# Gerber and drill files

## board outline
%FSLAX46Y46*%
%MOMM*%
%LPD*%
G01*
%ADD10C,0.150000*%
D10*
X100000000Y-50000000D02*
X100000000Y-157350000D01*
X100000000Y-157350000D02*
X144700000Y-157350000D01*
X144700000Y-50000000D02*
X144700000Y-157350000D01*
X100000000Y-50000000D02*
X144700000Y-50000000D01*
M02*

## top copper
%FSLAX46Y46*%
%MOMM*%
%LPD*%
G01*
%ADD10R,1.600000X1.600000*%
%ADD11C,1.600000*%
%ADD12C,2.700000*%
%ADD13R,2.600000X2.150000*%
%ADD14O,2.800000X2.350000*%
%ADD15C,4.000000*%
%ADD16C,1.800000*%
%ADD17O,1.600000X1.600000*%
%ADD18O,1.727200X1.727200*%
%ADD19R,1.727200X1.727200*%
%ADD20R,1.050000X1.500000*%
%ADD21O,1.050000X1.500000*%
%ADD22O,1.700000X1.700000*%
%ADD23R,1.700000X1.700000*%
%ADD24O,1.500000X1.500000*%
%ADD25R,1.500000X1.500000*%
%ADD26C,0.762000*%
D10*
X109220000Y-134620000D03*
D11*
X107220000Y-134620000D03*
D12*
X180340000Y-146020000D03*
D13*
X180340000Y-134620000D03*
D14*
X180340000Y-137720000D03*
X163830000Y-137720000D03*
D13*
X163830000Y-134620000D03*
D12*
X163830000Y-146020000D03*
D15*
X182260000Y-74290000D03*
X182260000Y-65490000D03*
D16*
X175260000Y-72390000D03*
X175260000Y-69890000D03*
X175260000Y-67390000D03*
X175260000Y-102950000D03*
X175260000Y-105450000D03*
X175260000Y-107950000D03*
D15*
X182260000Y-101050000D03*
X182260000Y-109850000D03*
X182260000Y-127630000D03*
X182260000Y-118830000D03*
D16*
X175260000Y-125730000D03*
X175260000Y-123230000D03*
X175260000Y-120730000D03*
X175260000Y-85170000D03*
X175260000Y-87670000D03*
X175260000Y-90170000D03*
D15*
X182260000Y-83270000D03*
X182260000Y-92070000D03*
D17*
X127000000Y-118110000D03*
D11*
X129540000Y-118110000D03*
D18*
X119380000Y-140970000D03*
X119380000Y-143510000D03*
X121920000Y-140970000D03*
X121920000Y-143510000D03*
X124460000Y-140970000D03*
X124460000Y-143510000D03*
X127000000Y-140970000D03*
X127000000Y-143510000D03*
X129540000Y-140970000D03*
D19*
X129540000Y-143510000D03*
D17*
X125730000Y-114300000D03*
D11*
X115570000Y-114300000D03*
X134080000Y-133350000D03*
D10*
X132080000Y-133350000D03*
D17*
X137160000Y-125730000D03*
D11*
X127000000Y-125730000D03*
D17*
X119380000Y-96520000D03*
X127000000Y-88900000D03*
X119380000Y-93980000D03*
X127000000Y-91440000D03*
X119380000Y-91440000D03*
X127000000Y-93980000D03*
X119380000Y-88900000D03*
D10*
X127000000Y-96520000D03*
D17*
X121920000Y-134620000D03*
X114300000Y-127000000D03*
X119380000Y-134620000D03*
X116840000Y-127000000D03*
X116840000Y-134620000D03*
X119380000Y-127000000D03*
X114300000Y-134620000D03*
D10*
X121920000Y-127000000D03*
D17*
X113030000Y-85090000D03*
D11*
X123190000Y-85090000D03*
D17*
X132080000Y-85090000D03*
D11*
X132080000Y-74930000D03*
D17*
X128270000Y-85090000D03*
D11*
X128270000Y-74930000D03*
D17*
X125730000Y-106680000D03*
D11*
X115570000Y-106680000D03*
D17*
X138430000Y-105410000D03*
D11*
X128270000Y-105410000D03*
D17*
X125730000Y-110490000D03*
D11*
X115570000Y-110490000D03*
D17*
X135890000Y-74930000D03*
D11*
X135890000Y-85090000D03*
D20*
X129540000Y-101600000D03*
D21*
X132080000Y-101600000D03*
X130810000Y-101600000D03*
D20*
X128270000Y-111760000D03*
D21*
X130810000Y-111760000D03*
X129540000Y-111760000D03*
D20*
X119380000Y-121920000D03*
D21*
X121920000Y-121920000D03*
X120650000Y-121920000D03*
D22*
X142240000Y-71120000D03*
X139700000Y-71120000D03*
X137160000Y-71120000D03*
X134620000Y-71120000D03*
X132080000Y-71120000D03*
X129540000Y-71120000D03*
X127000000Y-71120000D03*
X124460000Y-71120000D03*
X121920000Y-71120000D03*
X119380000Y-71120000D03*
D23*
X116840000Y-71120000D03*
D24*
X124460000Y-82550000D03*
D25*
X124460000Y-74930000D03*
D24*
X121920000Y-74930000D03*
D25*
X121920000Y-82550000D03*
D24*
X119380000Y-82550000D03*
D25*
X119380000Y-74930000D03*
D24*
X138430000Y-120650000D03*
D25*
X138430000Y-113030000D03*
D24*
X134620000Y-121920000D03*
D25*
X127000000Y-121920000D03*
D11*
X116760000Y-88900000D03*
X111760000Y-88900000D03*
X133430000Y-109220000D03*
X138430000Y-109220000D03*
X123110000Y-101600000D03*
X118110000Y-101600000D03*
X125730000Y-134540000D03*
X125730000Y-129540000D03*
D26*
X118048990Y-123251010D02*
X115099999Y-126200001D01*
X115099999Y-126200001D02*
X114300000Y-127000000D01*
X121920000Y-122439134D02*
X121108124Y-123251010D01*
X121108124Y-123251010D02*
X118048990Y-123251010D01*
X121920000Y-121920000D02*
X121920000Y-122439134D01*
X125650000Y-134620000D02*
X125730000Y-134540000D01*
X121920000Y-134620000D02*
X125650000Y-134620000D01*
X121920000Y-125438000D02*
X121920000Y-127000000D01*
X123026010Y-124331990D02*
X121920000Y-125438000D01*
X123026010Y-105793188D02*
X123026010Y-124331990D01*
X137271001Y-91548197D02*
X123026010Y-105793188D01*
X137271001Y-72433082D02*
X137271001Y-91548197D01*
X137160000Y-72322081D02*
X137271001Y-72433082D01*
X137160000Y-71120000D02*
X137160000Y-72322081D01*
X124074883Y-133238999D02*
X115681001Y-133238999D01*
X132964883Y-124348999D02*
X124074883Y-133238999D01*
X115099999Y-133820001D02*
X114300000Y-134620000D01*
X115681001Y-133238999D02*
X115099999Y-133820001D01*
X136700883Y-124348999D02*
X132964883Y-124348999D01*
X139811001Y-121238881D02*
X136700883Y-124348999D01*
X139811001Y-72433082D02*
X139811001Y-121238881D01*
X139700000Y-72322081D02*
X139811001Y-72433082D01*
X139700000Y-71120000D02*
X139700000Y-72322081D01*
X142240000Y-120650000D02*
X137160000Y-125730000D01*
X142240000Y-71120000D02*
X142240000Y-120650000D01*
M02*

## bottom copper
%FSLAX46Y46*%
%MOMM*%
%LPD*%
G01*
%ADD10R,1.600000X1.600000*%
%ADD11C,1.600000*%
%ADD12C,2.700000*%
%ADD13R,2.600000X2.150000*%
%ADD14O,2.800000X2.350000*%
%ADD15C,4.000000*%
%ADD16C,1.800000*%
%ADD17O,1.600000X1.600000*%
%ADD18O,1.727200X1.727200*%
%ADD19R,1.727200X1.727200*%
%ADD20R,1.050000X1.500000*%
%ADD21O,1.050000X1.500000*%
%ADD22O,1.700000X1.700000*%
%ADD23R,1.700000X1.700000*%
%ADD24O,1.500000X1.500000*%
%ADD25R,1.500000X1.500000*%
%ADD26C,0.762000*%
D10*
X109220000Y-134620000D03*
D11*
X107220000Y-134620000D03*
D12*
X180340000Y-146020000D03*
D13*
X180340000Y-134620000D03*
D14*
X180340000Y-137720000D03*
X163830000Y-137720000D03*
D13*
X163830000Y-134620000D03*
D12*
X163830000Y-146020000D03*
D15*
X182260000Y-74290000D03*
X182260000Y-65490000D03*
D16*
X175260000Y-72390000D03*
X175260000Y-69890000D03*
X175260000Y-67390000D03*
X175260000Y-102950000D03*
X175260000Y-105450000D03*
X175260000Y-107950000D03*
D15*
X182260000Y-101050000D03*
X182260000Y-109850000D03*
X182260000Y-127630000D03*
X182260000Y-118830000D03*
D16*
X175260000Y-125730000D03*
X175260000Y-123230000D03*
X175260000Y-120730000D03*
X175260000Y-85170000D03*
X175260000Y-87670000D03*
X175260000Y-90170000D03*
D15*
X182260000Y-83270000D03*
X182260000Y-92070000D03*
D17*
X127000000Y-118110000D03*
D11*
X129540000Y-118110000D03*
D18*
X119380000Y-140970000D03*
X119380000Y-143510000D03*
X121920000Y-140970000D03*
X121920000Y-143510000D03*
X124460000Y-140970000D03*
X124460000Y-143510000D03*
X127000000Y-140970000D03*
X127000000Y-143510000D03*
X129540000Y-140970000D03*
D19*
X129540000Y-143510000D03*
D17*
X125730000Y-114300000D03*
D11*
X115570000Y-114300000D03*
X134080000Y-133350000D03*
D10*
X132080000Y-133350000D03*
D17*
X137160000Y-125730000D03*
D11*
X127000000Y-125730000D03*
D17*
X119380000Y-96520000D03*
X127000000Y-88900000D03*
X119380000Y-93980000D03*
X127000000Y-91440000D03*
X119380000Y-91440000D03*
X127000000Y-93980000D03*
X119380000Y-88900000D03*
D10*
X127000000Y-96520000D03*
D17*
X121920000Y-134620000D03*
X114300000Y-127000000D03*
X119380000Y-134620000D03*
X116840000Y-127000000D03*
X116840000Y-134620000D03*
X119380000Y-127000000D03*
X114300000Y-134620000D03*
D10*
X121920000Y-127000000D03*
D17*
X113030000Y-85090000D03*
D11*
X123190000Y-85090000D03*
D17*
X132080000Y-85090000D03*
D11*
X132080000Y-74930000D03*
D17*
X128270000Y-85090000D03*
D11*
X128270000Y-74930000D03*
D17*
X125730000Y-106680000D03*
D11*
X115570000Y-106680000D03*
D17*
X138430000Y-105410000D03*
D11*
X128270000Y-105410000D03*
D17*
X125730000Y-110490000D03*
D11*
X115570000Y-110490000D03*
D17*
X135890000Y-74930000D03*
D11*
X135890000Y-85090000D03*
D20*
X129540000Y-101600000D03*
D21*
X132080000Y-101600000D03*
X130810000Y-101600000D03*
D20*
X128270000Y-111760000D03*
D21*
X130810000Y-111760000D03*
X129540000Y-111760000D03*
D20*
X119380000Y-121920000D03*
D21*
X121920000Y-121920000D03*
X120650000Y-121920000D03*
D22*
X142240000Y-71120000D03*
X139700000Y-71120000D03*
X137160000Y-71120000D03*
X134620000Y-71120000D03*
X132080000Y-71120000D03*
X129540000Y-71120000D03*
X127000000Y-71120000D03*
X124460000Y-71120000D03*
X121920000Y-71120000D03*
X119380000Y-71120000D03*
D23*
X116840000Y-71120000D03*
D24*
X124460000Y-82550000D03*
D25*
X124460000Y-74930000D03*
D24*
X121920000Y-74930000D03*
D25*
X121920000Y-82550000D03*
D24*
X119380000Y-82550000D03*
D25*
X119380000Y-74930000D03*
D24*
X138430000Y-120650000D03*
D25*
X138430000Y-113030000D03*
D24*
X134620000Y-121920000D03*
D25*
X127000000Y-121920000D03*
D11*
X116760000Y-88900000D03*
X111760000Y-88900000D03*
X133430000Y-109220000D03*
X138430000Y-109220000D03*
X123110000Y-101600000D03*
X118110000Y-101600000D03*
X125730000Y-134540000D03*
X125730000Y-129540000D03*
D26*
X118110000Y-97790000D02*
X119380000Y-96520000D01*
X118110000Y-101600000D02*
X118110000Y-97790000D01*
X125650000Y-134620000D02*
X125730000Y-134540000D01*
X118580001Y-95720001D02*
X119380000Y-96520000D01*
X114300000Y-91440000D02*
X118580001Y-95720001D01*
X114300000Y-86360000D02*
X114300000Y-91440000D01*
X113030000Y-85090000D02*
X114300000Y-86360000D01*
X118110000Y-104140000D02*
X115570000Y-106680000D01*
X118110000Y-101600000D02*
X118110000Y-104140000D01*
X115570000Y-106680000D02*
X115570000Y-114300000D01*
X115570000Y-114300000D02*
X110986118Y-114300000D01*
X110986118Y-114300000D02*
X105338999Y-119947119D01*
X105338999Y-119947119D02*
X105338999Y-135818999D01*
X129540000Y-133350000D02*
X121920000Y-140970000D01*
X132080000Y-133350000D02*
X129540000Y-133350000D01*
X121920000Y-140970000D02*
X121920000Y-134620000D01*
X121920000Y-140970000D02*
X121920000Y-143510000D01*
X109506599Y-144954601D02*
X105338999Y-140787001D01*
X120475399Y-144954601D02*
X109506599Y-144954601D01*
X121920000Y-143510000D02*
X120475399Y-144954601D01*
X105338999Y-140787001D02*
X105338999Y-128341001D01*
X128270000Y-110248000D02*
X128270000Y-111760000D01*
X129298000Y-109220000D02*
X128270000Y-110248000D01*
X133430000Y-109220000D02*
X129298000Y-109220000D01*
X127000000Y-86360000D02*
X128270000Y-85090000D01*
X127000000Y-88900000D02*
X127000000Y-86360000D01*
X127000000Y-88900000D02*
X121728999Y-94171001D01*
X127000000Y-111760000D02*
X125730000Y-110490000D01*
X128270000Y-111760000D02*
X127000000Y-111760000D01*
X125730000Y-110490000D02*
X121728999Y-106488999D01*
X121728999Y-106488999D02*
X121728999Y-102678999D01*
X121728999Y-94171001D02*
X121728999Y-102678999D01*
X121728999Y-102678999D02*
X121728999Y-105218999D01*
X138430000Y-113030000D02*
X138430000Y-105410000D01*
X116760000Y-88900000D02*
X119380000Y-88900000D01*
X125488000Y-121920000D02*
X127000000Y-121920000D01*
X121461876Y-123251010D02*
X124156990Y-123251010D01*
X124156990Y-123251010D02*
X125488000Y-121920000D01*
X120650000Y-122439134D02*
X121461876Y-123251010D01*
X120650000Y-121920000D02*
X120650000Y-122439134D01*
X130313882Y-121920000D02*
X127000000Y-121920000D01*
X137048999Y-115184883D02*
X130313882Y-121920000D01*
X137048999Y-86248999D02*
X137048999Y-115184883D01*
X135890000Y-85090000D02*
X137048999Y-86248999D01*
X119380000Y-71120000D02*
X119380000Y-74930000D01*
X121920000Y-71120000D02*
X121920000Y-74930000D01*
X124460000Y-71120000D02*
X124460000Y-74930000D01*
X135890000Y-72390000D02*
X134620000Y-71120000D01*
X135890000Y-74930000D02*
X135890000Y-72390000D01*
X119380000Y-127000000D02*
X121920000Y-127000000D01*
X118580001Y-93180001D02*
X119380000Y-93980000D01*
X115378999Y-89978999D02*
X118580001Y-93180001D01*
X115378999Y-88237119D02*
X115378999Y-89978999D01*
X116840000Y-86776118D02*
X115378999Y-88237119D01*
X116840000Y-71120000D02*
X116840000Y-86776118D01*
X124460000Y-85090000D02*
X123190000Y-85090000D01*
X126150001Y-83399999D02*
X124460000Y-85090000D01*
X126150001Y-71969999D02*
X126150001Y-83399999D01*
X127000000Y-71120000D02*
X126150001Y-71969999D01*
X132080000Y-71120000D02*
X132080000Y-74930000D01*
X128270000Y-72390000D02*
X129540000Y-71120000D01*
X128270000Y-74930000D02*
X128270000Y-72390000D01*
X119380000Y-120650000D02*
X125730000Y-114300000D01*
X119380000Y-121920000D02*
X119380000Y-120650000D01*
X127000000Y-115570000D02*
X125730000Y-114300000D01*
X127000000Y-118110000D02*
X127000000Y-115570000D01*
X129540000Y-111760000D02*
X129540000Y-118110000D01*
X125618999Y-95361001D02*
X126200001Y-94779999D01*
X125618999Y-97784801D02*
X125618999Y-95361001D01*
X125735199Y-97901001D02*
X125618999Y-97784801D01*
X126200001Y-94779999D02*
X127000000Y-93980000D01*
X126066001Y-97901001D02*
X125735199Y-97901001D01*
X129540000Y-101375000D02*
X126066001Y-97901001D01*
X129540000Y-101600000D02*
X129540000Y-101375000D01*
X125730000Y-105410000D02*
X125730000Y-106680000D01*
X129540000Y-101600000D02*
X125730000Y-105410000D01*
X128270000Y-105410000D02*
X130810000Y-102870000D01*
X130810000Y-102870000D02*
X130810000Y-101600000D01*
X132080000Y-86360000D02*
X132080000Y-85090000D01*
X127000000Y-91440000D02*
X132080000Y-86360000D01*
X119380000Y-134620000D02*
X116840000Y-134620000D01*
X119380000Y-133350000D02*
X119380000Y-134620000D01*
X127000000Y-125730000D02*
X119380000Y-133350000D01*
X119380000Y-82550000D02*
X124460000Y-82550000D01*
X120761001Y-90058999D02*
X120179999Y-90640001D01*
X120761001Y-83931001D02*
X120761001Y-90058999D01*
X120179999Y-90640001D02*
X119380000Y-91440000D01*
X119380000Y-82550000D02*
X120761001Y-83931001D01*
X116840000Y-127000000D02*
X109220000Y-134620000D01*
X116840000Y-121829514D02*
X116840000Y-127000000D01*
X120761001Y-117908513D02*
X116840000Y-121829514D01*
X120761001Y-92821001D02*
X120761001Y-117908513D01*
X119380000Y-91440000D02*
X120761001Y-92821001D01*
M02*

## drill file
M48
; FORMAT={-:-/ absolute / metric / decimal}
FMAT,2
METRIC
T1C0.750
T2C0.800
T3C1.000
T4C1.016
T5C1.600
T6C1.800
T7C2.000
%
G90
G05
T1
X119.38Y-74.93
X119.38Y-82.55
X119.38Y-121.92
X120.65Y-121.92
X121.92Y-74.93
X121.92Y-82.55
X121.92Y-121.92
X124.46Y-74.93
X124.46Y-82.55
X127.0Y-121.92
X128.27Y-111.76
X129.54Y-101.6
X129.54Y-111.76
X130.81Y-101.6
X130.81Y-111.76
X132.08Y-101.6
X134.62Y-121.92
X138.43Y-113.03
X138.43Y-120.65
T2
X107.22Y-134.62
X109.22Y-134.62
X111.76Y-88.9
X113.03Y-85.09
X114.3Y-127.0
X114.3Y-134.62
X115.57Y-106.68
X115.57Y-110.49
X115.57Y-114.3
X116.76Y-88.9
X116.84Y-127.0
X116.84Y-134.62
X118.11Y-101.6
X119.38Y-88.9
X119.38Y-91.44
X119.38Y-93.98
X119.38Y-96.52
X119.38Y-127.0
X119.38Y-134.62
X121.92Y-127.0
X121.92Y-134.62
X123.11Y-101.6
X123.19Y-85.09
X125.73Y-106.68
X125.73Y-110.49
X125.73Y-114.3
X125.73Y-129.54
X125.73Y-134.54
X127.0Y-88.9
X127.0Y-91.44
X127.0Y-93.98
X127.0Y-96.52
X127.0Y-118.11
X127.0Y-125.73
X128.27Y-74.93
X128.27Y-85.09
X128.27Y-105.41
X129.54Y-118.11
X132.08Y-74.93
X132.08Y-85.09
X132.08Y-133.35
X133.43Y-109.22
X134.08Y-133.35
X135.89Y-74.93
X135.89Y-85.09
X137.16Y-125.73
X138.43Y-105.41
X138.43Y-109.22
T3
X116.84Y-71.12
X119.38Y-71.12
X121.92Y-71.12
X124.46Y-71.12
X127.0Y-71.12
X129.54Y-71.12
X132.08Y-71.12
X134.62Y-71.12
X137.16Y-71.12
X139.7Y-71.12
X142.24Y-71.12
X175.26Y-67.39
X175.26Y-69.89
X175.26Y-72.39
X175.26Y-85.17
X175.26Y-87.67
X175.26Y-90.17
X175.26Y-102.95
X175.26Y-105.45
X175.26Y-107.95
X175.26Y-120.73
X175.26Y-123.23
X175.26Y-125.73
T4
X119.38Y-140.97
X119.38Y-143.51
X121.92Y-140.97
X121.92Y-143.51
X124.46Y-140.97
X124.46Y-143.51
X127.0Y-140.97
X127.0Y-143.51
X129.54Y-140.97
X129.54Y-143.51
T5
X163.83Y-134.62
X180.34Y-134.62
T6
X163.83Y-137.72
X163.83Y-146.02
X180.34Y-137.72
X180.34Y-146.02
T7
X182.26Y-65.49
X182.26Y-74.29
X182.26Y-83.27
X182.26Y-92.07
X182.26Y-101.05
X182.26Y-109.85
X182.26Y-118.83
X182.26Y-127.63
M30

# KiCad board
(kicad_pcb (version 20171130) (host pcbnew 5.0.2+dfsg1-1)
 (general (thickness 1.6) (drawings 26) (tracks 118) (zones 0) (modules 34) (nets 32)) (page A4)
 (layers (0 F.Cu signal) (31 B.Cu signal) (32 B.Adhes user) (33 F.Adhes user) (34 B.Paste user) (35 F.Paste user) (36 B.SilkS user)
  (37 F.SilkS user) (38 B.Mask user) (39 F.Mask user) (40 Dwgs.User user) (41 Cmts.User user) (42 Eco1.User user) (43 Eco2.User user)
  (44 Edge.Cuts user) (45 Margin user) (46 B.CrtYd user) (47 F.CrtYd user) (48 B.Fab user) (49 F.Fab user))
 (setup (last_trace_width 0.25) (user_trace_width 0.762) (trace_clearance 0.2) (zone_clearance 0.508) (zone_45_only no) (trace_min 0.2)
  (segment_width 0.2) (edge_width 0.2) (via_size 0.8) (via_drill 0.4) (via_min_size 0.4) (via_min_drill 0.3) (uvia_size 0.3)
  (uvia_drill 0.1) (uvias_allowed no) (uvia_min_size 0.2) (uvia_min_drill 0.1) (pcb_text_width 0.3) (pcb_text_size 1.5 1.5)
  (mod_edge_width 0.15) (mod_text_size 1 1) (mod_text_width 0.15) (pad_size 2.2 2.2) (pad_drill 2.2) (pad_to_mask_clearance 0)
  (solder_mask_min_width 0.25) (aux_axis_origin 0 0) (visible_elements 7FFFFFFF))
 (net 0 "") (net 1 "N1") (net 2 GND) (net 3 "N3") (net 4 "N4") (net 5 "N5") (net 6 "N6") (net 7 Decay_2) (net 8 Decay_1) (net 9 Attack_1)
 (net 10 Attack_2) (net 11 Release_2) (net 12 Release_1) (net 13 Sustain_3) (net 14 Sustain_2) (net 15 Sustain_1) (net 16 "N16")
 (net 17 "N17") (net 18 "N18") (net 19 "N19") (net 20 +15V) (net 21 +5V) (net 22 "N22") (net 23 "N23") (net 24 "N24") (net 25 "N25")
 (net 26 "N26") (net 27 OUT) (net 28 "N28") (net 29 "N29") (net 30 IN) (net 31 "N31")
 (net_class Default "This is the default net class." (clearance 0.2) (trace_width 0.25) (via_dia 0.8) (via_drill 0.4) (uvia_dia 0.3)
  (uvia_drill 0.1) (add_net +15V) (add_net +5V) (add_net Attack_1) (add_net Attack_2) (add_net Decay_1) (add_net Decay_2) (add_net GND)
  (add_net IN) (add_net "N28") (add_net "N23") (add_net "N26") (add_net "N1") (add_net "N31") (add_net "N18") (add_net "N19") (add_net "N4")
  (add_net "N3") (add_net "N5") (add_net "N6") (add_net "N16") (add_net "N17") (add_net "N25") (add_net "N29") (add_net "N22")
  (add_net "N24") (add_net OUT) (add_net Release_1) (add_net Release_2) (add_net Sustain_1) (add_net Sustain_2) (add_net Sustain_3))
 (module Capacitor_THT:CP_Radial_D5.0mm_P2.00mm (layer F.Cu) (at 109.22 134.62 180)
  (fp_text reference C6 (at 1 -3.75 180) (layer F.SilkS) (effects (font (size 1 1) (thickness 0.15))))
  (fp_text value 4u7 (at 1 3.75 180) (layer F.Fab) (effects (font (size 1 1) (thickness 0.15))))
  (pad 1 thru_hole rect (at 0 0 180) (size 1.6 1.6) (drill 0.8) (layers *.Cu *.Mask) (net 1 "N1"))
  (pad 2 thru_hole circle (at 2 0 180) (size 1.6 1.6) (drill 0.8) (layers *.Cu *.Mask) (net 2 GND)))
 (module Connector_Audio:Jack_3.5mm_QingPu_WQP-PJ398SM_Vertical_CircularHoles (layer F.Cu) (at 180.34 134.62)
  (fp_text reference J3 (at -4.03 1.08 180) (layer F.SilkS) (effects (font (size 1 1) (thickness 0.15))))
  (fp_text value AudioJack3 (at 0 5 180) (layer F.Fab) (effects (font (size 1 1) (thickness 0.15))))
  (pad T thru_hole circle (at 0 11.4 180) (size 2.7 2.7) (drill 1.8) (layers *.Cu *.Mask) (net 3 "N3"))
  (pad S thru_hole rect (at 0 0 180) (size 2.6 2.15) (drill 1.6) (layers *.Cu *.Mask) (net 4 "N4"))
  (pad TN thru_hole oval (at 0 3.1 180) (size 2.8 2.35) (drill 1.8) (layers *.Cu *.Mask)))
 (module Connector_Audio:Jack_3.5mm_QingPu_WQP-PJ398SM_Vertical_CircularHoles (layer F.Cu) (at 163.83 134.62)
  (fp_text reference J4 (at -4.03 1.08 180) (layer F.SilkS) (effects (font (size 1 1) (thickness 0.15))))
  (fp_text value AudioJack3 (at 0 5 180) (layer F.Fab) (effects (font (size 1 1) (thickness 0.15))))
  (pad TN thru_hole oval (at 0 3.1 180) (size 2.8 2.35) (drill 1.8) (layers *.Cu *.Mask))
  (pad S thru_hole rect (at 0 0 180) (size 2.6 2.15) (drill 1.6) (layers *.Cu *.Mask) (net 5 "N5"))
  (pad T thru_hole circle (at 0 11.4 180) (size 2.7 2.7) (drill 1.8) (layers *.Cu *.Mask) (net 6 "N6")))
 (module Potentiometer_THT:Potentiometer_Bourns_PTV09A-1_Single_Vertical (layer F.Cu) (at 175.26 72.39)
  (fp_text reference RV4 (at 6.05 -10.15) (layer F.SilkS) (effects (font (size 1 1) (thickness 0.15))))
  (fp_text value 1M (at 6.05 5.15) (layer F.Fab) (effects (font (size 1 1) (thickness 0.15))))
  (pad "" np_thru_hole circle (at 7 1.9) (size 4 4) (drill 2) (layers *.Cu *.Mask))
  (pad "" np_thru_hole circle (at 7 -6.9) (size 4 4) (drill 2) (layers *.Cu *.Mask))
  (pad 1 thru_hole circle (at 0 0) (size 1.8 1.8) (drill 1) (layers *.Cu *.Mask) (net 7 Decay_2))
  (pad 2 thru_hole circle (at 0 -2.5) (size 1.8 1.8) (drill 1) (layers *.Cu *.Mask) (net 7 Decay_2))
  (pad 3 thru_hole circle (at 0 -5) (size 1.8 1.8) (drill 1) (layers *.Cu *.Mask) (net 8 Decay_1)))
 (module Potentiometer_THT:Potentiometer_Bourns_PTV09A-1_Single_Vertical (layer F.Cu) (at 175.26 107.95)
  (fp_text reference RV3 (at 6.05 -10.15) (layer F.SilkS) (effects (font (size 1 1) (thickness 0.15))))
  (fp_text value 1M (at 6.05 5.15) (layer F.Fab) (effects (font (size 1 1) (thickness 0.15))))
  (pad 3 thru_hole circle (at 0 -5) (size 1.8 1.8) (drill 1) (layers *.Cu *.Mask) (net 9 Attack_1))
  (pad 2 thru_hole circle (at 0 -2.5) (size 1.8 1.8) (drill 1) (layers *.Cu *.Mask) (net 9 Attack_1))
  (pad 1 thru_hole circle (at 0 0) (size 1.8 1.8) (drill 1) (layers *.Cu *.Mask) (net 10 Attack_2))
  (pad "" np_thru_hole circle (at 7 -6.9) (size 4 4) (drill 2) (layers *.Cu *.Mask))
  (pad "" np_thru_hole circle (at 7 1.9) (size 4 4) (drill 2) (layers *.Cu *.Mask)))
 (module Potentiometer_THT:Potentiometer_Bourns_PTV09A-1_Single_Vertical (layer F.Cu) (at 175.26 125.73)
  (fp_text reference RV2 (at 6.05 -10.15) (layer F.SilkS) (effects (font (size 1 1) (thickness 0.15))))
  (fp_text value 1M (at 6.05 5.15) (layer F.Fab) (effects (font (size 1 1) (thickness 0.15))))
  (pad "" np_thru_hole circle (at 7 1.9) (size 4 4) (drill 2) (layers *.Cu *.Mask))
  (pad "" np_thru_hole circle (at 7 -6.9) (size 4 4) (drill 2) (layers *.Cu *.Mask))
  (pad 1 thru_hole circle (at 0 0) (size 1.8 1.8) (drill 1) (layers *.Cu *.Mask) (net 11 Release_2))
  (pad 2 thru_hole circle (at 0 -2.5) (size 1.8 1.8) (drill 1) (layers *.Cu *.Mask) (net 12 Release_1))
  (pad 3 thru_hole circle (at 0 -5) (size 1.8 1.8) (drill 1) (layers *.Cu *.Mask) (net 12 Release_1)))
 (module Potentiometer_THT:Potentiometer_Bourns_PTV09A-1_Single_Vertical (layer F.Cu) (at 175.26 90.17)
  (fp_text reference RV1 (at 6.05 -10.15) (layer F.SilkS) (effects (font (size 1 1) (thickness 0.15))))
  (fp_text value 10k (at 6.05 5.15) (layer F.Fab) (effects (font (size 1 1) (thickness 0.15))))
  (pad 3 thru_hole circle (at 0 -5) (size 1.8 1.8) (drill 1) (layers *.Cu *.Mask) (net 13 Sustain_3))
  (pad 2 thru_hole circle (at 0 -2.5) (size 1.8 1.8) (drill 1) (layers *.Cu *.Mask) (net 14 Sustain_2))
  (pad 1 thru_hole circle (at 0 0) (size 1.8 1.8) (drill 1) (layers *.Cu *.Mask) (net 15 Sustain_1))
  (pad "" np_thru_hole circle (at 7 -6.9) (size 4 4) (drill 2) (layers *.Cu *.Mask))
  (pad "" np_thru_hole circle (at 7 1.9) (size 4 4) (drill 2) (layers *.Cu *.Mask)))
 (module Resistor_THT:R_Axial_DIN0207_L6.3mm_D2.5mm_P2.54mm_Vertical (layer F.Cu) (at 129.54 118.11 180)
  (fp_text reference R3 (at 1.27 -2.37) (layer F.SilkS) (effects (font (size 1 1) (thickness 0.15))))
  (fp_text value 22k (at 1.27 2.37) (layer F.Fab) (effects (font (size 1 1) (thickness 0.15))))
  (pad 2 thru_hole oval (at 2.54 0 180) (size 1.6 1.6) (drill 0.8) (layers *.Cu *.Mask) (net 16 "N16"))
  (pad 1 thru_hole circle (at 0 0 180) (size 1.6 1.6) (drill 0.8) (layers *.Cu *.Mask) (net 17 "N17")))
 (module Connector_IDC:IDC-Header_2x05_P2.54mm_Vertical (layer B.Cu) (at 129.54 143.51 90)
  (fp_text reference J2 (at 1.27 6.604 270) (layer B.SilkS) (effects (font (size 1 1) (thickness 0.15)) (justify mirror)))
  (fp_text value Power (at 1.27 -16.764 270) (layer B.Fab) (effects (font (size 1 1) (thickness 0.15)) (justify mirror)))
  (pad 10 thru_hole oval (at 2.54 -10.16 90) (size 1.7272 1.7272) (drill 1.016) (layers *.Cu *.Mask) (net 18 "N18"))
  (pad 9 thru_hole oval (at 0 -10.16 90) (size 1.7272 1.7272) (drill 1.016) (layers *.Cu *.Mask) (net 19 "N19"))
  (pad 8 thru_hole oval (at 2.54 -7.62 90) (size 1.7272 1.7272) (drill 1.016) (layers *.Cu *.Mask) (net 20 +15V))
  (pad 7 thru_hole oval (at 0 -7.62 90) (size 1.7272 1.7272) (drill 1.016) (layers *.Cu *.Mask) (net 20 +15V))
  (pad 6 thru_hole oval (at 2.54 -5.08 90) (size 1.7272 1.7272) (drill 1.016) (layers *.Cu *.Mask) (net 2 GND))
  (pad 5 thru_hole oval (at 0 -5.08 90) (size 1.7272 1.7272) (drill 1.016) (layers *.Cu *.Mask) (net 2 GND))
  (pad 4 thru_hole oval (at 2.54 -2.54 90) (size 1.7272 1.7272) (drill 1.016) (layers *.Cu *.Mask) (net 2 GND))
  (pad 3 thru_hole oval (at 0 -2.54 90) (size 1.7272 1.7272) (drill 1.016) (layers *.Cu *.Mask) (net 2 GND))
  (pad 2 thru_hole oval (at 2.54 0 90) (size 1.7272 1.7272) (drill 1.016) (layers *.Cu *.Mask) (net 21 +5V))
  (pad 1 thru_hole rect (at 0 0 90) (size 1.7272 1.7272) (drill 1.016) (layers *.Cu *.Mask) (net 21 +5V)))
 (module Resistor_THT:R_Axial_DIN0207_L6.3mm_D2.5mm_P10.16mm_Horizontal (layer F.Cu) (at 115.57 114.3)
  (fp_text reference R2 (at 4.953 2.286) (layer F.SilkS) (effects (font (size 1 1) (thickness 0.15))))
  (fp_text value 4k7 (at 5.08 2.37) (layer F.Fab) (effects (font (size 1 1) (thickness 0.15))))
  (pad 2 thru_hole oval (at 10.16 0) (size 1.6 1.6) (drill 0.8) (layers *.Cu *.Mask) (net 16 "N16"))
  (pad 1 thru_hole circle (at 0 0) (size 1.6 1.6) (drill 0.8) (layers *.Cu *.Mask) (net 20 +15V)))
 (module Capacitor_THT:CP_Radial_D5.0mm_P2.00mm (layer F.Cu) (at 132.08 133.35)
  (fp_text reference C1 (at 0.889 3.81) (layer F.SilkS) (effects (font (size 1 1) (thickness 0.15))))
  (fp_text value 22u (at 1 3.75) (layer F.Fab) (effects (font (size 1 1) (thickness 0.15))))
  (pad 2 thru_hole circle (at 2 0) (size 1.6 1.6) (drill 0.8) (layers *.Cu *.Mask) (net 2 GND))
  (pad 1 thru_hole rect (at 0 0) (size 1.6 1.6) (drill 0.8) (layers *.Cu *.Mask) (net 20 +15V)))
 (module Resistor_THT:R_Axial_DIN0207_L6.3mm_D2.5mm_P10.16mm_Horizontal (layer F.Cu) (at 127 125.73)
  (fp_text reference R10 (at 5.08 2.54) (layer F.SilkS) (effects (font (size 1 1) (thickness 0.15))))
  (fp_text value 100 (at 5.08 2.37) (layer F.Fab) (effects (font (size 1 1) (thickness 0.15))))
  (pad 2 thru_hole oval (at 10.16 0) (size 1.6 1.6) (drill 0.8) (layers *.Cu *.Mask) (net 7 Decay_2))
  (pad 1 thru_hole circle (at 0 0) (size 1.6 1.6) (drill 0.8) (layers *.Cu *.Mask) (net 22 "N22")))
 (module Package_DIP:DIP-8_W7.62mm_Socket (layer F.Cu) (at 127 96.52 180)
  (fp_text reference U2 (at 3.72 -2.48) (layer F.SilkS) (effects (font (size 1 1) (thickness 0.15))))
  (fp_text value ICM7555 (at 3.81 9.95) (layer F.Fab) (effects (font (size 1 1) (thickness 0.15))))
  (pad 8 thru_hole oval (at 7.62 0 180) (size 1.6 1.6) (drill 0.8) (layers *.Cu *.Mask) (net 20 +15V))
  (pad 4 thru_hole oval (at 0 7.62 180) (size 1.6 1.6) (drill 0.8) (layers *.Cu *.Mask) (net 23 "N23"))
  (pad 7 thru_hole oval (at 7.62 2.54 180) (size 1.6 1.6) (drill 0.8) (layers *.Cu *.Mask) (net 13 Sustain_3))
  (pad 3 thru_hole oval (at 0 5.08 180) (size 1.6 1.6) (drill 0.8) (layers *.Cu *.Mask) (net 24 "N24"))
  (pad 6 thru_hole oval (at 7.62 5.08 180) (size 1.6 1.6) (drill 0.8) (layers *.Cu *.Mask) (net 1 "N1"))
  (pad 2 thru_hole oval (at 0 2.54 180) (size 1.6 1.6) (drill 0.8) (layers *.Cu *.Mask) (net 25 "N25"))
  (pad 5 thru_hole oval (at 7.62 7.62 180) (size 1.6 1.6) (drill 0.8) (layers *.Cu *.Mask) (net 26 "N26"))
  (pad 1 thru_hole rect (at 0 0 180) (size 1.6 1.6) (drill 0.8) (layers *.Cu *.Mask) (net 2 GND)))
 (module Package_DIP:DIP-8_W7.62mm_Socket (layer F.Cu) (at 121.92 127 270)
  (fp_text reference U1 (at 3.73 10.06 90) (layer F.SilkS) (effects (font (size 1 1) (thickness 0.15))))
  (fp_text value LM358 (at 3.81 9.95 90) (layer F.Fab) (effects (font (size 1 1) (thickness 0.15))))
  (pad 8 thru_hole oval (at 7.62 0 270) (size 1.6 1.6) (drill 0.8) (layers *.Cu *.Mask) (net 20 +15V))
  (pad 4 thru_hole oval (at 0 7.62 270) (size 1.6 1.6) (drill 0.8) (layers *.Cu *.Mask) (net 2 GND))
  (pad 7 thru_hole oval (at 7.62 2.54 270) (size 1.6 1.6) (drill 0.8) (layers *.Cu *.Mask) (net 22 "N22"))
  (pad 3 thru_hole oval (at 0 5.08 270) (size 1.6 1.6) (drill 0.8) (layers *.Cu *.Mask) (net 1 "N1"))
  (pad 6 thru_hole oval (at 7.62 5.08 270) (size 1.6 1.6) (drill 0.8) (layers *.Cu *.Mask) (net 22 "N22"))
  (pad 2 thru_hole oval (at 0 2.54 270) (size 1.6 1.6) (drill 0.8) (layers *.Cu *.Mask) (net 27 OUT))
  (pad 5 thru_hole oval (at 7.62 7.62 270) (size 1.6 1.6) (drill 0.8) (layers *.Cu *.Mask) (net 14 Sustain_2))
  (pad 1 thru_hole rect (at 0 0 270) (size 1.6 1.6) (drill 0.8) (layers *.Cu *.Mask) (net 27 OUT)))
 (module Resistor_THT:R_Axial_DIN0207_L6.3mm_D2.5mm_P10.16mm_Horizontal (layer F.Cu) (at 123.19 85.09 180)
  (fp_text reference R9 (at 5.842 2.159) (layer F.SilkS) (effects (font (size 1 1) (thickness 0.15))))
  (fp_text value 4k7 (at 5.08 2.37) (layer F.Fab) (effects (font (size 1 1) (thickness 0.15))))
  (pad 2 thru_hole oval (at 10.16 0 180) (size 1.6 1.6) (drill 0.8) (layers *.Cu *.Mask) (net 20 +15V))
  (pad 1 thru_hole circle (at 0 0 180) (size 1.6 1.6) (drill 0.8) (layers *.Cu *.Mask) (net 15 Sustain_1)))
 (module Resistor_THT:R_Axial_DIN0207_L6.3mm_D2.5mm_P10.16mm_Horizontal (layer F.Cu) (at 132.08 74.93 270)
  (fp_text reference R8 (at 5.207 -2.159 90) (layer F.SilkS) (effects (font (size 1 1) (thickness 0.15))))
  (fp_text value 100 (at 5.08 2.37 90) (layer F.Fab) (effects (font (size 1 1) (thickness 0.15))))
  (pad 2 thru_hole oval (at 10.16 0 270) (size 1.6 1.6) (drill 0.8) (layers *.Cu *.Mask) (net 24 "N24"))
  (pad 1 thru_hole circle (at 0 0 270) (size 1.6 1.6) (drill 0.8) (layers *.Cu *.Mask) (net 9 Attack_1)))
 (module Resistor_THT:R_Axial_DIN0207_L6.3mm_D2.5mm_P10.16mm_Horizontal (layer F.Cu) (at 128.27 74.93 270)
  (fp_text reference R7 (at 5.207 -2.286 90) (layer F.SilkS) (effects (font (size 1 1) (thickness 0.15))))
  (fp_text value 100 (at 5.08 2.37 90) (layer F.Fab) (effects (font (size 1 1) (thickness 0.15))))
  (pad 2 thru_hole oval (at 10.16 0 270) (size 1.6 1.6) (drill 0.8) (layers *.Cu *.Mask) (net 23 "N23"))
  (pad 1 thru_hole circle (at 0 0 270) (size 1.6 1.6) (drill 0.8) (layers *.Cu *.Mask) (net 12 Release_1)))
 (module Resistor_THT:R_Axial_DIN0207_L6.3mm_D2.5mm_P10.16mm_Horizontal (layer F.Cu) (at 115.57 106.68)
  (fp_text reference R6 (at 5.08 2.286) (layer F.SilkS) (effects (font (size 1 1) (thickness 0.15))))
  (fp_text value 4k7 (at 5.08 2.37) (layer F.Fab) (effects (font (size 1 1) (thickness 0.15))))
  (pad 2 thru_hole oval (at 10.16 0) (size 1.6 1.6) (drill 0.8) (layers *.Cu *.Mask) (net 25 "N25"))
  (pad 1 thru_hole circle (at 0 0) (size 1.6 1.6) (drill 0.8) (layers *.Cu *.Mask) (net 20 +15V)))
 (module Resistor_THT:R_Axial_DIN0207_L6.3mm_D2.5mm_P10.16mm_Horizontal (layer F.Cu) (at 128.27 105.41)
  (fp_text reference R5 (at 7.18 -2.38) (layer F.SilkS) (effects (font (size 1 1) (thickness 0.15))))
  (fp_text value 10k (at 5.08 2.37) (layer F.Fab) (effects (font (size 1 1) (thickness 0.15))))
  (pad 2 thru_hole oval (at 10.16 0) (size 1.6 1.6) (drill 0.8) (layers *.Cu *.Mask) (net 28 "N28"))
  (pad 1 thru_hole circle (at 0 0) (size 1.6 1.6) (drill 0.8) (layers *.Cu *.Mask) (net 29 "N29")))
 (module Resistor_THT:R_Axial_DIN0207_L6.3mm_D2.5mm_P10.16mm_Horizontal (layer F.Cu) (at 115.57 110.49)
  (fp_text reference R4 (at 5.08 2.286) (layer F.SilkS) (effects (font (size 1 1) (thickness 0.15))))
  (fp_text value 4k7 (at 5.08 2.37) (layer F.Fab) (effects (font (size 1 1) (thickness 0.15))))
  (pad 2 thru_hole oval (at 10.16 0) (size 1.6 1.6) (drill 0.8) (layers *.Cu *.Mask) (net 23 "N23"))
  (pad 1 thru_hole circle (at 0 0) (size 1.6 1.6) (drill 0.8) (layers *.Cu *.Mask) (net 20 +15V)))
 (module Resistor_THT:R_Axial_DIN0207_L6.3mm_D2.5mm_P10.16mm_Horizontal (layer F.Cu) (at 135.89 85.09 90)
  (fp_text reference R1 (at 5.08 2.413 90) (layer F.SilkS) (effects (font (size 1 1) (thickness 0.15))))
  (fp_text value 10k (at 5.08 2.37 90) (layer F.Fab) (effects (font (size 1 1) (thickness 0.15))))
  (pad 2 thru_hole oval (at 10.16 0 90) (size 1.6 1.6) (drill 0.8) (layers *.Cu *.Mask) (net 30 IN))
  (pad 1 thru_hole circle (at 0 0 90) (size 1.6 1.6) (drill 0.8) (layers *.Cu *.Mask) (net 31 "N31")))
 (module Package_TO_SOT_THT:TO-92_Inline (layer F.Cu) (at 129.54 101.6)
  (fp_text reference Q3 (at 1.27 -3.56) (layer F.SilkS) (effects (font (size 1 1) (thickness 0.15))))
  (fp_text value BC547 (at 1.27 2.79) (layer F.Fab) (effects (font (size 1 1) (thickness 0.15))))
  (pad 1 thru_hole rect (at 0 0) (size 1.05 1.5) (drill 0.75) (layers *.Cu *.Mask) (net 25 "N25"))
  (pad 3 thru_hole oval (at 2.54 0) (size 1.05 1.5) (drill 0.75) (layers *.Cu *.Mask) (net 2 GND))
  (pad 2 thru_hole oval (at 1.27 0) (size 1.05 1.5) (drill 0.75) (layers *.Cu *.Mask) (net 29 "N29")))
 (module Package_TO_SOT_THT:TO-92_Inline (layer F.Cu) (at 128.27 111.76)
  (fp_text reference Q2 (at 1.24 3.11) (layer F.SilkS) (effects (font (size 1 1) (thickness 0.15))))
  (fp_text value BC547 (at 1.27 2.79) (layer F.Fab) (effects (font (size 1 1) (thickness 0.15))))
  (pad 1 thru_hole rect (at 0 0) (size 1.05 1.5) (drill 0.75) (layers *.Cu *.Mask) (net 23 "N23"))
  (pad 3 thru_hole oval (at 2.54 0) (size 1.05 1.5) (drill 0.75) (layers *.Cu *.Mask) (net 2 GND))
  (pad 2 thru_hole oval (at 1.27 0) (size 1.05 1.5) (drill 0.75) (layers *.Cu *.Mask) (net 17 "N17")))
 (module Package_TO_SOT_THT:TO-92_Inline (layer F.Cu) (at 119.38 121.92)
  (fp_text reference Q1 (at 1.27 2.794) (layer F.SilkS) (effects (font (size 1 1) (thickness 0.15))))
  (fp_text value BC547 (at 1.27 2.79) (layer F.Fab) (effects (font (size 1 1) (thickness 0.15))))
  (pad 1 thru_hole rect (at 0 0) (size 1.05 1.5) (drill 0.75) (layers *.Cu *.Mask) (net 16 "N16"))
  (pad 3 thru_hole oval (at 2.54 0) (size 1.05 1.5) (drill 0.75) (layers *.Cu *.Mask) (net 2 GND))
  (pad 2 thru_hole oval (at 1.27 0) (size 1.05 1.5) (drill 0.75) (layers *.Cu *.Mask) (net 31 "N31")))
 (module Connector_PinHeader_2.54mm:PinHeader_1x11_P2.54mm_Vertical (layer B.Cu) (at 116.84 71.12 270)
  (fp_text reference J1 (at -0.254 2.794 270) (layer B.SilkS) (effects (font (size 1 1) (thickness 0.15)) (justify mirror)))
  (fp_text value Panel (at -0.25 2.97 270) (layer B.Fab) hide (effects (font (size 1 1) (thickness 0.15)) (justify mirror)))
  (pad 11 thru_hole oval (at 0 -25.4 270) (size 1.7 1.7) (drill 1) (layers *.Cu *.Mask) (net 7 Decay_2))
  (pad 10 thru_hole oval (at 0 -22.86 270) (size 1.7 1.7) (drill 1) (layers *.Cu *.Mask) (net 14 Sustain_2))
  (pad 9 thru_hole oval (at 0 -20.32 270) (size 1.7 1.7) (drill 1) (layers *.Cu *.Mask) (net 27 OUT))
  (pad 8 thru_hole oval (at 0 -17.78 270) (size 1.7 1.7) (drill 1) (layers *.Cu *.Mask) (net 30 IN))
  (pad 7 thru_hole oval (at 0 -15.24 270) (size 1.7 1.7) (drill 1) (layers *.Cu *.Mask) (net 9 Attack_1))
  (pad 6 thru_hole oval (at 0 -12.7 270) (size 1.7 1.7) (drill 1) (layers *.Cu *.Mask) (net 12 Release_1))
  (pad 5 thru_hole oval (at 0 -10.16 270) (size 1.7 1.7) (drill 1) (layers *.Cu *.Mask) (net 15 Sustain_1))
  (pad 4 thru_hole oval (at 0 -7.62 270) (size 1.7 1.7) (drill 1) (layers *.Cu *.Mask) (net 8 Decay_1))
  (pad 3 thru_hole oval (at 0 -5.08 270) (size 1.7 1.7) (drill 1) (layers *.Cu *.Mask) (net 10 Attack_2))
  (pad 2 thru_hole oval (at 0 -2.54 270) (size 1.7 1.7) (drill 1) (layers *.Cu *.Mask) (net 11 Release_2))
  (pad 1 thru_hole rect (at 0 0 270) (size 1.7 1.7) (drill 1) (layers *.Cu *.Mask) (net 13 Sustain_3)))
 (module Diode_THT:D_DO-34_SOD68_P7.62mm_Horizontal (layer F.Cu) (at 124.46 74.93 270)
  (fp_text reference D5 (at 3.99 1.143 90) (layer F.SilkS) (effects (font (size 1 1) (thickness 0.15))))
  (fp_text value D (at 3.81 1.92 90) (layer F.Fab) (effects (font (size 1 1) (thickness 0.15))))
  (pad 2 thru_hole oval (at 7.62 0 270) (size 1.5 1.5) (drill 0.75) (layers *.Cu *.Mask) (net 1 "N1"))
  (pad 1 thru_hole rect (at 0 0 270) (size 1.5 1.5) (drill 0.75) (layers *.Cu *.Mask) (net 8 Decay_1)))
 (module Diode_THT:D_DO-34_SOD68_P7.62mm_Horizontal (layer F.Cu) (at 121.92 82.55 90)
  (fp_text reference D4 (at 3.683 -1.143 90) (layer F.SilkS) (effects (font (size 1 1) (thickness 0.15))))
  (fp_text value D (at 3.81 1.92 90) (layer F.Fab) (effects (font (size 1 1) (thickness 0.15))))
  (pad 2 thru_hole oval (at 7.62 0 90) (size 1.5 1.5) (drill 0.75) (layers *.Cu *.Mask) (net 10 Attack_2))
  (pad 1 thru_hole rect (at 0 0 90) (size 1.5 1.5) (drill 0.75) (layers *.Cu *.Mask) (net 1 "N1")))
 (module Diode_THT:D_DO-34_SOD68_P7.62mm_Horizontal (layer F.Cu) (at 119.38 74.93 270)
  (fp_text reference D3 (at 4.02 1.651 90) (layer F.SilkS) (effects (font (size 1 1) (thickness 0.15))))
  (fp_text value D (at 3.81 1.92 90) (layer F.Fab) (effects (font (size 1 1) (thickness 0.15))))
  (pad 2 thru_hole oval (at 7.62 0 270) (size 1.5 1.5) (drill 0.75) (layers *.Cu *.Mask) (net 1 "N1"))
  (pad 1 thru_hole rect (at 0 0 270) (size 1.5 1.5) (drill 0.75) (layers *.Cu *.Mask) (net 11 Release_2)))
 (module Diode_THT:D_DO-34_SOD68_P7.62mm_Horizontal (layer F.Cu) (at 138.43 113.03 270)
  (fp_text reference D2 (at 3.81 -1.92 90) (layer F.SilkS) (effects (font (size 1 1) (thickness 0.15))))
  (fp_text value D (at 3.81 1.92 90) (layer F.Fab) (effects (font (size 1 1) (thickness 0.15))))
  (pad 2 thru_hole oval (at 7.62 0 270) (size 1.5 1.5) (drill 0.75) (layers *.Cu *.Mask) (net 2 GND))
  (pad 1 thru_hole rect (at 0 0 270) (size 1.5 1.5) (drill 0.75) (layers *.Cu *.Mask) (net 28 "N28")))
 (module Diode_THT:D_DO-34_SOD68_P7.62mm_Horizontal (layer F.Cu) (at 127 121.92)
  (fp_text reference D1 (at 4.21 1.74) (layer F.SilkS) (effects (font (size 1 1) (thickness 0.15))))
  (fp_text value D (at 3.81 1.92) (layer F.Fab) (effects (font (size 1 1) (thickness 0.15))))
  (pad 2 thru_hole oval (at 7.62 0) (size 1.5 1.5) (drill 0.75) (layers *.Cu *.Mask) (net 2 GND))
  (pad 1 thru_hole rect (at 0 0) (size 1.5 1.5) (drill 0.75) (layers *.Cu *.Mask) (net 31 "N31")))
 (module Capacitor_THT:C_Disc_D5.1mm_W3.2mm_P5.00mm (layer F.Cu) (at 111.76 88.9)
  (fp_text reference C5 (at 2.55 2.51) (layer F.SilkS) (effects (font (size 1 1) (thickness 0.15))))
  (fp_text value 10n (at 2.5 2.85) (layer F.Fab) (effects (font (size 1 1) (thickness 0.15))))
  (pad 2 thru_hole circle (at 5 0) (size 1.6 1.6) (drill 0.8) (layers *.Cu *.Mask) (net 26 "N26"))
  (pad 1 thru_hole circle (at 0 0) (size 1.6 1.6) (drill 0.8) (layers *.Cu *.Mask) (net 2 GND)))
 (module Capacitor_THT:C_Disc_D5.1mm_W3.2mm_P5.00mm (layer F.Cu) (at 138.43 109.22 180)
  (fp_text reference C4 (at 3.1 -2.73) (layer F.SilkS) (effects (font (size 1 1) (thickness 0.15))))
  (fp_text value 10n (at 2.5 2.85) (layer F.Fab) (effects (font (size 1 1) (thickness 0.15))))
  (pad 2 thru_hole circle (at 5 0 180) (size 1.6 1.6) (drill 0.8) (layers *.Cu *.Mask) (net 23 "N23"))
  (pad 1 thru_hole circle (at 0 0 180) (size 1.6 1.6) (drill 0.8) (layers *.Cu *.Mask) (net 28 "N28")))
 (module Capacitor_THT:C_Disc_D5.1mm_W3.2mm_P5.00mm (layer F.Cu) (at 118.11 101.6)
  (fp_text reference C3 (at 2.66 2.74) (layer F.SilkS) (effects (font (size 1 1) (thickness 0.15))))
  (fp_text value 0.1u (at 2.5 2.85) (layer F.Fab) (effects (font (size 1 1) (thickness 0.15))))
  (pad 2 thru_hole circle (at 5 0) (size 1.6 1.6) (drill 0.8) (layers *.Cu *.Mask) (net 2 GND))
  (pad 1 thru_hole circle (at 0 0) (size 1.6 1.6) (drill 0.8) (layers *.Cu *.Mask) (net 20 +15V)))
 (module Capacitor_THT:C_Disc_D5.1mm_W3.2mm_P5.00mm (layer F.Cu) (at 125.73 129.54 270)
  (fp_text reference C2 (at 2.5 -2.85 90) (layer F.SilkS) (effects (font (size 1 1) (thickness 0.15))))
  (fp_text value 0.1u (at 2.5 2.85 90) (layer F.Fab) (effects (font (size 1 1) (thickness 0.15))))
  (pad 2 thru_hole circle (at 5 0 270) (size 1.6 1.6) (drill 0.8) (layers *.Cu *.Mask) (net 20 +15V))
  (pad 1 thru_hole circle (at 0 0 270) (size 1.6 1.6) (drill 0.8) (layers *.Cu *.Mask) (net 2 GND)))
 (gr_line (start 100 50) (end 100 157.35) (layer Edge.Cuts) (width 0.15))
 (gr_line (start 100 157.35) (end 144.7 157.35) (layer Edge.Cuts) (width 0.15))
 (gr_line (start 144.7 50) (end 144.7 157.35) (layer Edge.Cuts) (width 0.15))
 (gr_line (start 100 50) (end 144.7 50) (layer Edge.Cuts) (width 0.15))
 (segment (start 118.04899 123.25101) (end 115.099999 126.200001) (width 0.762) (layer F.Cu) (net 2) (status 20))
 (segment (start 115.099999 126.200001) (end 114.3 127) (width 0.762) (layer F.Cu) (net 2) (status 30))
 (segment (start 121.92 122.439134) (end 121.108124 123.25101) (width 0.762) (layer F.Cu) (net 2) (status 10))
 (segment (start 121.108124 123.25101) (end 118.04899 123.25101) (width 0.762) (layer F.Cu) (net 2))
 (segment (start 121.92 121.92) (end 121.92 122.439134) (width 0.762) (layer F.Cu) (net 2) (status 30))
 (segment (start 118.11 97.79) (end 119.38 96.52) (width 0.762) (layer B.Cu) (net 20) (status 20))
 (segment (start 118.11 101.6) (end 118.11 97.79) (width 0.762) (layer B.Cu) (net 20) (status 10))
 (segment (start 125.65 134.62) (end 125.73 134.54) (width 0.762) (layer B.Cu) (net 20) (status 30))
 (segment (start 125.65 134.62) (end 125.73 134.54) (width 0.762) (layer F.Cu) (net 20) (status 30))
 (segment (start 121.92 134.62) (end 125.65 134.62) (width 0.762) (layer F.Cu) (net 20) (status 30))
 (segment (start 118.580001 95.720001) (end 119.38 96.52) (width 0.762) (layer B.Cu) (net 20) (status 30))
 (segment (start 114.3 91.44) (end 118.580001 95.720001) (width 0.762) (layer B.Cu) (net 20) (status 20))
 (segment (start 114.3 86.36) (end 114.3 91.44) (width 0.762) (layer B.Cu) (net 20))
 (segment (start 113.03 85.09) (end 114.3 86.36) (width 0.762) (layer B.Cu) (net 20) (status 10))
 (segment (start 118.11 104.14) (end 115.57 106.68) (width 0.762) (layer B.Cu) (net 20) (status 20))
 (segment (start 118.11 101.6) (end 118.11 104.14) (width 0.762) (layer B.Cu) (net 20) (status 10))
 (segment (start 115.57 106.68) (end 115.57 114.3) (width 0.762) (layer B.Cu) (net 20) (status 30))
 (segment (start 115.57 114.3) (end 110.986118 114.3) (width 0.762) (layer B.Cu) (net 20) (status 10))
 (segment (start 110.986118 114.3) (end 105.338999 119.947119) (width 0.762) (layer B.Cu) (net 20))
 (segment (start 105.338999 119.947119) (end 105.338999 135.818999) (width 0.762) (layer B.Cu) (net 20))
 (segment (start 129.54 133.35) (end 121.92 140.97) (width 0.762) (layer B.Cu) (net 20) (status 20))
 (segment (start 132.08 133.35) (end 129.54 133.35) (width 0.762) (layer B.Cu) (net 20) (status 10))
 (segment (start 121.92 140.97) (end 121.92 134.62) (width 0.762) (layer B.Cu) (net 20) (status 30))
 (segment (start 121.92 140.97) (end 121.92 143.51) (width 0.762) (layer B.Cu) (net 20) (status 30))
 (segment (start 109.506599 144.954601) (end 105.338999 140.787001) (width 0.762) (layer B.Cu) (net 20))
 (segment (start 120.475399 144.954601) (end 109.506599 144.954601) (width 0.762) (layer B.Cu) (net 20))
 (segment (start 121.92 143.51) (end 120.475399 144.954601) (width 0.762) (layer B.Cu) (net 20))
 (segment (start 105.338999 140.787001) (end 105.338999 128.341001) (width 0.762) (layer B.Cu) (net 20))
 (segment (start 128.27 110.248) (end 128.27 111.76) (width 0.762) (layer B.Cu) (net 23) (status 20))
 (segment (start 129.298 109.22) (end 128.27 110.248) (width 0.762) (layer B.Cu) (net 23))
 (segment (start 133.43 109.22) (end 129.298 109.22) (width 0.762) (layer B.Cu) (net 23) (status 10))
 (segment (start 127 86.36) (end 128.27 85.09) (width 0.762) (layer B.Cu) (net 23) (status 20))
 (segment (start 127 88.9) (end 127 86.36) (width 0.762) (layer B.Cu) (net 23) (status 10))
 (segment (start 127 88.9) (end 121.728999 94.171001) (width 0.762) (layer B.Cu) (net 23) (status 10))
 (segment (start 127 111.76) (end 125.73 110.49) (width 0.762) (layer B.Cu) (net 23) (status 20))
 (segment (start 128.27 111.76) (end 127 111.76) (width 0.762) (layer B.Cu) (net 23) (status 10))
 (segment (start 125.73 110.49) (end 121.728999 106.488999) (width 0.762) (layer B.Cu) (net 23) (status 10))
 (segment (start 121.728999 106.488999) (end 121.728999 102.678999) (width 0.762) (layer B.Cu) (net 23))
 (segment (start 121.728999 94.171001) (end 121.728999 102.678999) (width 0.762) (layer B.Cu) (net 23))
 (segment (start 121.728999 102.678999) (end 121.728999 105.218999) (width 0.762) (layer B.Cu) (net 23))
 (segment (start 138.43 113.03) (end 138.43 105.41) (width 0.762) (layer B.Cu) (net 28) (status 30))
 (segment (start 116.76 88.9) (end 119.38 88.9) (width 0.762) (layer B.Cu) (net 26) (status 30))
 (segment (start 125.488 121.92) (end 127 121.92) (width 0.762) (layer B.Cu) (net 31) (status 20))
 (segment (start 121.461876 123.25101) (end 124.15699 123.25101) (width 0.762) (layer B.Cu) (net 31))
 (segment (start 124.15699 123.25101) (end 125.488 121.92) (width 0.762) (layer B.Cu) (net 31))
 (segment (start 120.65 122.439134) (end 121.461876 123.25101) (width 0.762) (layer B.Cu) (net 31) (status 10))
 (segment (start 120.65 121.92) (end 120.65 122.439134) (width 0.762) (layer B.Cu) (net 31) (status 30))
 (segment (start 130.313882 121.92) (end 127 121.92) (width 0.762) (layer B.Cu) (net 31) (status 20))
 (segment (start 137.048999 115.184883) (end 130.313882 121.92) (width 0.762) (layer B.Cu) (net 31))
 (segment (start 137.048999 86.248999) (end 137.048999 115.184883) (width 0.762) (layer B.Cu) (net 31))
 (segment (start 135.89 85.09) (end 137.048999 86.248999) (width 0.762) (layer B.Cu) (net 31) (status 10))
 (segment (start 119.38 71.12) (end 119.38 74.93) (width 0.762) (layer B.Cu) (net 11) (status 30))
 (segment (start 121.92 71.12) (end 121.92 74.93) (width 0.762) (layer B.Cu) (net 10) (status 30))
 (segment (start 124.46 71.12) (end 124.46 74.93) (width 0.762) (layer B.Cu) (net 8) (status 30))
 (segment (start 135.89 72.39) (end 134.62 71.12) (width 0.762) (layer B.Cu) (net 30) (status 20))
 (segment (start 135.89 74.93) (end 135.89 72.39) (width 0.762) (layer B.Cu) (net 30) (status 10))
 (segment (start 119.38 127) (end 121.92 127) (width 0.762) (layer B.Cu) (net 27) (status 30))
 (segment (start 121.92 125.438) (end 121.92 127) (width 0.762) (layer F.Cu) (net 27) (status 20))
 (segment (start 123.02601 124.33199) (end 121.92 125.438) (width 0.762) (layer F.Cu) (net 27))
 (segment (start 123.02601 105.793188) (end 123.02601 124.33199) (width 0.762) (layer F.Cu) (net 27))
 (segment (start 137.271001 91.548197) (end 123.02601 105.793188) (width 0.762) (layer F.Cu) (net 27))
 (segment (start 137.271001 72.433082) (end 137.271001 91.548197) (width 0.762) (layer F.Cu) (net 27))
 (segment (start 137.16 72.322081) (end 137.271001 72.433082) (width 0.762) (layer F.Cu) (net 27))
 (segment (start 137.16 71.12) (end 137.16 72.322081) (width 0.762) (layer F.Cu) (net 27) (status 10))
 (segment (start 118.580001 93.180001) (end 119.38 93.98) (width 0.762) (layer B.Cu) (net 13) (status 30))
 (segment (start 115.378999 89.978999) (end 118.580001 93.180001) (width 0.762) (layer B.Cu) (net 13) (status 20))
 (segment (start 115.378999 88.237119) (end 115.378999 89.978999) (width 0.762) (layer B.Cu) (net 13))
 (segment (start 116.84 86.776118) (end 115.378999 88.237119) (width 0.762) (layer B.Cu) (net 13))
 (segment (start 116.84 71.12) (end 116.84 86.776118) (width 0.762) (layer B.Cu) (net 13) (status 10))
 (segment (start 124.074883 133.238999) (end 115.681001 133.238999) (width 0.762) (layer F.Cu) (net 14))
 (segment (start 132.964883 124.348999) (end 124.074883 133.238999) (width 0.762) (layer F.Cu) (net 14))
 (segment (start 115.099999 133.820001) (end 114.3 134.62) (width 0.762) (layer F.Cu) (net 14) (status 30))
 (segment (start 115.681001 133.238999) (end 115.099999 133.820001) (width 0.762) (layer F.Cu) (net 14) (status 20))
 (segment (start 136.700883 124.348999) (end 132.964883 124.348999) (width 0.762) (layer F.Cu) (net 14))
 (segment (start 139.811001 121.238881) (end 136.700883 124.348999) (width 0.762) (layer F.Cu) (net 14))
 (segment (start 139.811001 72.433082) (end 139.811001 121.238881) (width 0.762) (layer F.Cu) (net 14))
 (segment (start 139.7 72.322081) (end 139.811001 72.433082) (width 0.762) (layer F.Cu) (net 14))
 (segment (start 139.7 71.12) (end 139.7 72.322081) (width 0.762) (layer F.Cu) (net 14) (status 10))
 (segment (start 124.46 85.09) (end 123.19 85.09) (width 0.762) (layer B.Cu) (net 15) (status 20))
 (segment (start 126.150001 83.399999) (end 124.46 85.09) (width 0.762) (layer B.Cu) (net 15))
 (segment (start 126.150001 71.969999) (end 126.150001 83.399999) (width 0.762) (layer B.Cu) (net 15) (status 10))
 (segment (start 127 71.12) (end 126.150001 71.969999) (width 0.762) (layer B.Cu) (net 15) (status 30))
 (segment (start 142.24 120.65) (end 137.16 125.73) (width 0.762) (layer F.Cu) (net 7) (status 20))
 (segment (start 142.24 71.12) (end 142.24 120.65) (width 0.762) (layer F.Cu) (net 7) (status 10))
 (segment (start 132.08 71.12) (end 132.08 74.93) (width 0.762) (layer B.Cu) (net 9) (status 30))
 (segment (start 128.27 72.39) (end 129.54 71.12) (width 0.762) (layer B.Cu) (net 12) (status 20))
 (segment (start 128.27 74.93) (end 128.27 72.39) (width 0.762) (layer B.Cu) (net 12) (status 10))
 (segment (start 119.38 120.65) (end 125.73 114.3) (width 0.762) (layer B.Cu) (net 16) (status 20))
 (segment (start 119.38 121.92) (end 119.38 120.65) (width 0.762) (layer B.Cu) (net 16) (status 10))
 (segment (start 127 115.57) (end 125.73 114.3) (width 0.762) (layer B.Cu) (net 16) (status 20))
 (segment (start 127 118.11) (end 127 115.57) (width 0.762) (layer B.Cu) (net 16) (status 10))
 (segment (start 129.54 111.76) (end 129.54 118.11) (width 0.762) (layer B.Cu) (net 17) (status 30))
 (segment (start 125.618999 95.361001) (end 126.200001 94.779999) (width 0.762) (layer B.Cu) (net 25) (status 20))
 (segment (start 125.618999 97.784801) (end 125.618999 95.361001) (width 0.762) (layer B.Cu) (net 25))
 (segment (start 125.735199 97.901001) (end 125.618999 97.784801) (width 0.762) (layer B.Cu) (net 25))
 (segment (start 126.200001 94.779999) (end 127 93.98) (width 0.762) (layer B.Cu) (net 25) (status 30))
 (segment (start 126.066001 97.901001) (end 125.735199 97.901001) (width 0.762) (layer B.Cu) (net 25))
 (segment (start 129.54 101.375) (end 126.066001 97.901001) (width 0.762) (layer B.Cu) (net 25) (status 10))
 (segment (start 129.54 101.6) (end 129.54 101.375) (width 0.762) (layer B.Cu) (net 25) (status 30))
 (segment (start 125.73 105.41) (end 125.73 106.68) (width 0.762) (layer B.Cu) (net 25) (status 20))
 (segment (start 129.54 101.6) (end 125.73 105.41) (width 0.762) (layer B.Cu) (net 25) (status 10))
 (segment (start 128.27 105.41) (end 130.81 102.87) (width 0.762) (layer B.Cu) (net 29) (status 10))
 (segment (start 130.81 102.87) (end 130.81 101.6) (width 0.762) (layer B.Cu) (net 29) (status 20))
 (segment (start 132.08 86.36) (end 132.08 85.09) (width 0.762) (layer B.Cu) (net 24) (status 20))
 (segment (start 127 91.44) (end 132.08 86.36) (width 0.762) (layer B.Cu) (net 24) (status 10))
 (segment (start 119.38 134.62) (end 116.84 134.62) (width 0.762) (layer B.Cu) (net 22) (status 30))
 (segment (start 119.38 133.35) (end 119.38 134.62) (width 0.762) (layer B.Cu) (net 22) (status 20))
 (segment (start 127 125.73) (end 119.38 133.35) (width 0.762) (layer B.Cu) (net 22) (status 10))
 (segment (start 119.38 82.55) (end 124.46 82.55) (width 0.762) (layer B.Cu) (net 1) (status 30))
 (segment (start 120.761001 90.058999) (end 120.179999 90.640001) (width 0.762) (layer B.Cu) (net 1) (status 20))
 (segment (start 120.761001 83.931001) (end 120.761001 90.058999) (width 0.762) (layer B.Cu) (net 1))
 (segment (start 120.179999 90.640001) (end 119.38 91.44) (width 0.762) (layer B.Cu) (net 1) (status 30))
 (segment (start 119.38 82.55) (end 120.761001 83.931001) (width 0.762) (layer B.Cu) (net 1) (status 10))
 (segment (start 116.84 127) (end 109.22 134.62) (width 0.762) (layer B.Cu) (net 1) (status 30))
 (segment (start 116.84 121.829514) (end 116.84 127) (width 0.762) (layer B.Cu) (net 1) (status 20))
 (segment (start 120.761001 117.908513) (end 116.84 121.829514) (width 0.762) (layer B.Cu) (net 1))
 (segment (start 120.761001 92.821001) (end 120.761001 117.908513) (width 0.762) (layer B.Cu) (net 1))
 (segment (start 119.38 91.44) (end 120.761001 92.821001) (width 0.762) (layer B.Cu) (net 1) (status 10)))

